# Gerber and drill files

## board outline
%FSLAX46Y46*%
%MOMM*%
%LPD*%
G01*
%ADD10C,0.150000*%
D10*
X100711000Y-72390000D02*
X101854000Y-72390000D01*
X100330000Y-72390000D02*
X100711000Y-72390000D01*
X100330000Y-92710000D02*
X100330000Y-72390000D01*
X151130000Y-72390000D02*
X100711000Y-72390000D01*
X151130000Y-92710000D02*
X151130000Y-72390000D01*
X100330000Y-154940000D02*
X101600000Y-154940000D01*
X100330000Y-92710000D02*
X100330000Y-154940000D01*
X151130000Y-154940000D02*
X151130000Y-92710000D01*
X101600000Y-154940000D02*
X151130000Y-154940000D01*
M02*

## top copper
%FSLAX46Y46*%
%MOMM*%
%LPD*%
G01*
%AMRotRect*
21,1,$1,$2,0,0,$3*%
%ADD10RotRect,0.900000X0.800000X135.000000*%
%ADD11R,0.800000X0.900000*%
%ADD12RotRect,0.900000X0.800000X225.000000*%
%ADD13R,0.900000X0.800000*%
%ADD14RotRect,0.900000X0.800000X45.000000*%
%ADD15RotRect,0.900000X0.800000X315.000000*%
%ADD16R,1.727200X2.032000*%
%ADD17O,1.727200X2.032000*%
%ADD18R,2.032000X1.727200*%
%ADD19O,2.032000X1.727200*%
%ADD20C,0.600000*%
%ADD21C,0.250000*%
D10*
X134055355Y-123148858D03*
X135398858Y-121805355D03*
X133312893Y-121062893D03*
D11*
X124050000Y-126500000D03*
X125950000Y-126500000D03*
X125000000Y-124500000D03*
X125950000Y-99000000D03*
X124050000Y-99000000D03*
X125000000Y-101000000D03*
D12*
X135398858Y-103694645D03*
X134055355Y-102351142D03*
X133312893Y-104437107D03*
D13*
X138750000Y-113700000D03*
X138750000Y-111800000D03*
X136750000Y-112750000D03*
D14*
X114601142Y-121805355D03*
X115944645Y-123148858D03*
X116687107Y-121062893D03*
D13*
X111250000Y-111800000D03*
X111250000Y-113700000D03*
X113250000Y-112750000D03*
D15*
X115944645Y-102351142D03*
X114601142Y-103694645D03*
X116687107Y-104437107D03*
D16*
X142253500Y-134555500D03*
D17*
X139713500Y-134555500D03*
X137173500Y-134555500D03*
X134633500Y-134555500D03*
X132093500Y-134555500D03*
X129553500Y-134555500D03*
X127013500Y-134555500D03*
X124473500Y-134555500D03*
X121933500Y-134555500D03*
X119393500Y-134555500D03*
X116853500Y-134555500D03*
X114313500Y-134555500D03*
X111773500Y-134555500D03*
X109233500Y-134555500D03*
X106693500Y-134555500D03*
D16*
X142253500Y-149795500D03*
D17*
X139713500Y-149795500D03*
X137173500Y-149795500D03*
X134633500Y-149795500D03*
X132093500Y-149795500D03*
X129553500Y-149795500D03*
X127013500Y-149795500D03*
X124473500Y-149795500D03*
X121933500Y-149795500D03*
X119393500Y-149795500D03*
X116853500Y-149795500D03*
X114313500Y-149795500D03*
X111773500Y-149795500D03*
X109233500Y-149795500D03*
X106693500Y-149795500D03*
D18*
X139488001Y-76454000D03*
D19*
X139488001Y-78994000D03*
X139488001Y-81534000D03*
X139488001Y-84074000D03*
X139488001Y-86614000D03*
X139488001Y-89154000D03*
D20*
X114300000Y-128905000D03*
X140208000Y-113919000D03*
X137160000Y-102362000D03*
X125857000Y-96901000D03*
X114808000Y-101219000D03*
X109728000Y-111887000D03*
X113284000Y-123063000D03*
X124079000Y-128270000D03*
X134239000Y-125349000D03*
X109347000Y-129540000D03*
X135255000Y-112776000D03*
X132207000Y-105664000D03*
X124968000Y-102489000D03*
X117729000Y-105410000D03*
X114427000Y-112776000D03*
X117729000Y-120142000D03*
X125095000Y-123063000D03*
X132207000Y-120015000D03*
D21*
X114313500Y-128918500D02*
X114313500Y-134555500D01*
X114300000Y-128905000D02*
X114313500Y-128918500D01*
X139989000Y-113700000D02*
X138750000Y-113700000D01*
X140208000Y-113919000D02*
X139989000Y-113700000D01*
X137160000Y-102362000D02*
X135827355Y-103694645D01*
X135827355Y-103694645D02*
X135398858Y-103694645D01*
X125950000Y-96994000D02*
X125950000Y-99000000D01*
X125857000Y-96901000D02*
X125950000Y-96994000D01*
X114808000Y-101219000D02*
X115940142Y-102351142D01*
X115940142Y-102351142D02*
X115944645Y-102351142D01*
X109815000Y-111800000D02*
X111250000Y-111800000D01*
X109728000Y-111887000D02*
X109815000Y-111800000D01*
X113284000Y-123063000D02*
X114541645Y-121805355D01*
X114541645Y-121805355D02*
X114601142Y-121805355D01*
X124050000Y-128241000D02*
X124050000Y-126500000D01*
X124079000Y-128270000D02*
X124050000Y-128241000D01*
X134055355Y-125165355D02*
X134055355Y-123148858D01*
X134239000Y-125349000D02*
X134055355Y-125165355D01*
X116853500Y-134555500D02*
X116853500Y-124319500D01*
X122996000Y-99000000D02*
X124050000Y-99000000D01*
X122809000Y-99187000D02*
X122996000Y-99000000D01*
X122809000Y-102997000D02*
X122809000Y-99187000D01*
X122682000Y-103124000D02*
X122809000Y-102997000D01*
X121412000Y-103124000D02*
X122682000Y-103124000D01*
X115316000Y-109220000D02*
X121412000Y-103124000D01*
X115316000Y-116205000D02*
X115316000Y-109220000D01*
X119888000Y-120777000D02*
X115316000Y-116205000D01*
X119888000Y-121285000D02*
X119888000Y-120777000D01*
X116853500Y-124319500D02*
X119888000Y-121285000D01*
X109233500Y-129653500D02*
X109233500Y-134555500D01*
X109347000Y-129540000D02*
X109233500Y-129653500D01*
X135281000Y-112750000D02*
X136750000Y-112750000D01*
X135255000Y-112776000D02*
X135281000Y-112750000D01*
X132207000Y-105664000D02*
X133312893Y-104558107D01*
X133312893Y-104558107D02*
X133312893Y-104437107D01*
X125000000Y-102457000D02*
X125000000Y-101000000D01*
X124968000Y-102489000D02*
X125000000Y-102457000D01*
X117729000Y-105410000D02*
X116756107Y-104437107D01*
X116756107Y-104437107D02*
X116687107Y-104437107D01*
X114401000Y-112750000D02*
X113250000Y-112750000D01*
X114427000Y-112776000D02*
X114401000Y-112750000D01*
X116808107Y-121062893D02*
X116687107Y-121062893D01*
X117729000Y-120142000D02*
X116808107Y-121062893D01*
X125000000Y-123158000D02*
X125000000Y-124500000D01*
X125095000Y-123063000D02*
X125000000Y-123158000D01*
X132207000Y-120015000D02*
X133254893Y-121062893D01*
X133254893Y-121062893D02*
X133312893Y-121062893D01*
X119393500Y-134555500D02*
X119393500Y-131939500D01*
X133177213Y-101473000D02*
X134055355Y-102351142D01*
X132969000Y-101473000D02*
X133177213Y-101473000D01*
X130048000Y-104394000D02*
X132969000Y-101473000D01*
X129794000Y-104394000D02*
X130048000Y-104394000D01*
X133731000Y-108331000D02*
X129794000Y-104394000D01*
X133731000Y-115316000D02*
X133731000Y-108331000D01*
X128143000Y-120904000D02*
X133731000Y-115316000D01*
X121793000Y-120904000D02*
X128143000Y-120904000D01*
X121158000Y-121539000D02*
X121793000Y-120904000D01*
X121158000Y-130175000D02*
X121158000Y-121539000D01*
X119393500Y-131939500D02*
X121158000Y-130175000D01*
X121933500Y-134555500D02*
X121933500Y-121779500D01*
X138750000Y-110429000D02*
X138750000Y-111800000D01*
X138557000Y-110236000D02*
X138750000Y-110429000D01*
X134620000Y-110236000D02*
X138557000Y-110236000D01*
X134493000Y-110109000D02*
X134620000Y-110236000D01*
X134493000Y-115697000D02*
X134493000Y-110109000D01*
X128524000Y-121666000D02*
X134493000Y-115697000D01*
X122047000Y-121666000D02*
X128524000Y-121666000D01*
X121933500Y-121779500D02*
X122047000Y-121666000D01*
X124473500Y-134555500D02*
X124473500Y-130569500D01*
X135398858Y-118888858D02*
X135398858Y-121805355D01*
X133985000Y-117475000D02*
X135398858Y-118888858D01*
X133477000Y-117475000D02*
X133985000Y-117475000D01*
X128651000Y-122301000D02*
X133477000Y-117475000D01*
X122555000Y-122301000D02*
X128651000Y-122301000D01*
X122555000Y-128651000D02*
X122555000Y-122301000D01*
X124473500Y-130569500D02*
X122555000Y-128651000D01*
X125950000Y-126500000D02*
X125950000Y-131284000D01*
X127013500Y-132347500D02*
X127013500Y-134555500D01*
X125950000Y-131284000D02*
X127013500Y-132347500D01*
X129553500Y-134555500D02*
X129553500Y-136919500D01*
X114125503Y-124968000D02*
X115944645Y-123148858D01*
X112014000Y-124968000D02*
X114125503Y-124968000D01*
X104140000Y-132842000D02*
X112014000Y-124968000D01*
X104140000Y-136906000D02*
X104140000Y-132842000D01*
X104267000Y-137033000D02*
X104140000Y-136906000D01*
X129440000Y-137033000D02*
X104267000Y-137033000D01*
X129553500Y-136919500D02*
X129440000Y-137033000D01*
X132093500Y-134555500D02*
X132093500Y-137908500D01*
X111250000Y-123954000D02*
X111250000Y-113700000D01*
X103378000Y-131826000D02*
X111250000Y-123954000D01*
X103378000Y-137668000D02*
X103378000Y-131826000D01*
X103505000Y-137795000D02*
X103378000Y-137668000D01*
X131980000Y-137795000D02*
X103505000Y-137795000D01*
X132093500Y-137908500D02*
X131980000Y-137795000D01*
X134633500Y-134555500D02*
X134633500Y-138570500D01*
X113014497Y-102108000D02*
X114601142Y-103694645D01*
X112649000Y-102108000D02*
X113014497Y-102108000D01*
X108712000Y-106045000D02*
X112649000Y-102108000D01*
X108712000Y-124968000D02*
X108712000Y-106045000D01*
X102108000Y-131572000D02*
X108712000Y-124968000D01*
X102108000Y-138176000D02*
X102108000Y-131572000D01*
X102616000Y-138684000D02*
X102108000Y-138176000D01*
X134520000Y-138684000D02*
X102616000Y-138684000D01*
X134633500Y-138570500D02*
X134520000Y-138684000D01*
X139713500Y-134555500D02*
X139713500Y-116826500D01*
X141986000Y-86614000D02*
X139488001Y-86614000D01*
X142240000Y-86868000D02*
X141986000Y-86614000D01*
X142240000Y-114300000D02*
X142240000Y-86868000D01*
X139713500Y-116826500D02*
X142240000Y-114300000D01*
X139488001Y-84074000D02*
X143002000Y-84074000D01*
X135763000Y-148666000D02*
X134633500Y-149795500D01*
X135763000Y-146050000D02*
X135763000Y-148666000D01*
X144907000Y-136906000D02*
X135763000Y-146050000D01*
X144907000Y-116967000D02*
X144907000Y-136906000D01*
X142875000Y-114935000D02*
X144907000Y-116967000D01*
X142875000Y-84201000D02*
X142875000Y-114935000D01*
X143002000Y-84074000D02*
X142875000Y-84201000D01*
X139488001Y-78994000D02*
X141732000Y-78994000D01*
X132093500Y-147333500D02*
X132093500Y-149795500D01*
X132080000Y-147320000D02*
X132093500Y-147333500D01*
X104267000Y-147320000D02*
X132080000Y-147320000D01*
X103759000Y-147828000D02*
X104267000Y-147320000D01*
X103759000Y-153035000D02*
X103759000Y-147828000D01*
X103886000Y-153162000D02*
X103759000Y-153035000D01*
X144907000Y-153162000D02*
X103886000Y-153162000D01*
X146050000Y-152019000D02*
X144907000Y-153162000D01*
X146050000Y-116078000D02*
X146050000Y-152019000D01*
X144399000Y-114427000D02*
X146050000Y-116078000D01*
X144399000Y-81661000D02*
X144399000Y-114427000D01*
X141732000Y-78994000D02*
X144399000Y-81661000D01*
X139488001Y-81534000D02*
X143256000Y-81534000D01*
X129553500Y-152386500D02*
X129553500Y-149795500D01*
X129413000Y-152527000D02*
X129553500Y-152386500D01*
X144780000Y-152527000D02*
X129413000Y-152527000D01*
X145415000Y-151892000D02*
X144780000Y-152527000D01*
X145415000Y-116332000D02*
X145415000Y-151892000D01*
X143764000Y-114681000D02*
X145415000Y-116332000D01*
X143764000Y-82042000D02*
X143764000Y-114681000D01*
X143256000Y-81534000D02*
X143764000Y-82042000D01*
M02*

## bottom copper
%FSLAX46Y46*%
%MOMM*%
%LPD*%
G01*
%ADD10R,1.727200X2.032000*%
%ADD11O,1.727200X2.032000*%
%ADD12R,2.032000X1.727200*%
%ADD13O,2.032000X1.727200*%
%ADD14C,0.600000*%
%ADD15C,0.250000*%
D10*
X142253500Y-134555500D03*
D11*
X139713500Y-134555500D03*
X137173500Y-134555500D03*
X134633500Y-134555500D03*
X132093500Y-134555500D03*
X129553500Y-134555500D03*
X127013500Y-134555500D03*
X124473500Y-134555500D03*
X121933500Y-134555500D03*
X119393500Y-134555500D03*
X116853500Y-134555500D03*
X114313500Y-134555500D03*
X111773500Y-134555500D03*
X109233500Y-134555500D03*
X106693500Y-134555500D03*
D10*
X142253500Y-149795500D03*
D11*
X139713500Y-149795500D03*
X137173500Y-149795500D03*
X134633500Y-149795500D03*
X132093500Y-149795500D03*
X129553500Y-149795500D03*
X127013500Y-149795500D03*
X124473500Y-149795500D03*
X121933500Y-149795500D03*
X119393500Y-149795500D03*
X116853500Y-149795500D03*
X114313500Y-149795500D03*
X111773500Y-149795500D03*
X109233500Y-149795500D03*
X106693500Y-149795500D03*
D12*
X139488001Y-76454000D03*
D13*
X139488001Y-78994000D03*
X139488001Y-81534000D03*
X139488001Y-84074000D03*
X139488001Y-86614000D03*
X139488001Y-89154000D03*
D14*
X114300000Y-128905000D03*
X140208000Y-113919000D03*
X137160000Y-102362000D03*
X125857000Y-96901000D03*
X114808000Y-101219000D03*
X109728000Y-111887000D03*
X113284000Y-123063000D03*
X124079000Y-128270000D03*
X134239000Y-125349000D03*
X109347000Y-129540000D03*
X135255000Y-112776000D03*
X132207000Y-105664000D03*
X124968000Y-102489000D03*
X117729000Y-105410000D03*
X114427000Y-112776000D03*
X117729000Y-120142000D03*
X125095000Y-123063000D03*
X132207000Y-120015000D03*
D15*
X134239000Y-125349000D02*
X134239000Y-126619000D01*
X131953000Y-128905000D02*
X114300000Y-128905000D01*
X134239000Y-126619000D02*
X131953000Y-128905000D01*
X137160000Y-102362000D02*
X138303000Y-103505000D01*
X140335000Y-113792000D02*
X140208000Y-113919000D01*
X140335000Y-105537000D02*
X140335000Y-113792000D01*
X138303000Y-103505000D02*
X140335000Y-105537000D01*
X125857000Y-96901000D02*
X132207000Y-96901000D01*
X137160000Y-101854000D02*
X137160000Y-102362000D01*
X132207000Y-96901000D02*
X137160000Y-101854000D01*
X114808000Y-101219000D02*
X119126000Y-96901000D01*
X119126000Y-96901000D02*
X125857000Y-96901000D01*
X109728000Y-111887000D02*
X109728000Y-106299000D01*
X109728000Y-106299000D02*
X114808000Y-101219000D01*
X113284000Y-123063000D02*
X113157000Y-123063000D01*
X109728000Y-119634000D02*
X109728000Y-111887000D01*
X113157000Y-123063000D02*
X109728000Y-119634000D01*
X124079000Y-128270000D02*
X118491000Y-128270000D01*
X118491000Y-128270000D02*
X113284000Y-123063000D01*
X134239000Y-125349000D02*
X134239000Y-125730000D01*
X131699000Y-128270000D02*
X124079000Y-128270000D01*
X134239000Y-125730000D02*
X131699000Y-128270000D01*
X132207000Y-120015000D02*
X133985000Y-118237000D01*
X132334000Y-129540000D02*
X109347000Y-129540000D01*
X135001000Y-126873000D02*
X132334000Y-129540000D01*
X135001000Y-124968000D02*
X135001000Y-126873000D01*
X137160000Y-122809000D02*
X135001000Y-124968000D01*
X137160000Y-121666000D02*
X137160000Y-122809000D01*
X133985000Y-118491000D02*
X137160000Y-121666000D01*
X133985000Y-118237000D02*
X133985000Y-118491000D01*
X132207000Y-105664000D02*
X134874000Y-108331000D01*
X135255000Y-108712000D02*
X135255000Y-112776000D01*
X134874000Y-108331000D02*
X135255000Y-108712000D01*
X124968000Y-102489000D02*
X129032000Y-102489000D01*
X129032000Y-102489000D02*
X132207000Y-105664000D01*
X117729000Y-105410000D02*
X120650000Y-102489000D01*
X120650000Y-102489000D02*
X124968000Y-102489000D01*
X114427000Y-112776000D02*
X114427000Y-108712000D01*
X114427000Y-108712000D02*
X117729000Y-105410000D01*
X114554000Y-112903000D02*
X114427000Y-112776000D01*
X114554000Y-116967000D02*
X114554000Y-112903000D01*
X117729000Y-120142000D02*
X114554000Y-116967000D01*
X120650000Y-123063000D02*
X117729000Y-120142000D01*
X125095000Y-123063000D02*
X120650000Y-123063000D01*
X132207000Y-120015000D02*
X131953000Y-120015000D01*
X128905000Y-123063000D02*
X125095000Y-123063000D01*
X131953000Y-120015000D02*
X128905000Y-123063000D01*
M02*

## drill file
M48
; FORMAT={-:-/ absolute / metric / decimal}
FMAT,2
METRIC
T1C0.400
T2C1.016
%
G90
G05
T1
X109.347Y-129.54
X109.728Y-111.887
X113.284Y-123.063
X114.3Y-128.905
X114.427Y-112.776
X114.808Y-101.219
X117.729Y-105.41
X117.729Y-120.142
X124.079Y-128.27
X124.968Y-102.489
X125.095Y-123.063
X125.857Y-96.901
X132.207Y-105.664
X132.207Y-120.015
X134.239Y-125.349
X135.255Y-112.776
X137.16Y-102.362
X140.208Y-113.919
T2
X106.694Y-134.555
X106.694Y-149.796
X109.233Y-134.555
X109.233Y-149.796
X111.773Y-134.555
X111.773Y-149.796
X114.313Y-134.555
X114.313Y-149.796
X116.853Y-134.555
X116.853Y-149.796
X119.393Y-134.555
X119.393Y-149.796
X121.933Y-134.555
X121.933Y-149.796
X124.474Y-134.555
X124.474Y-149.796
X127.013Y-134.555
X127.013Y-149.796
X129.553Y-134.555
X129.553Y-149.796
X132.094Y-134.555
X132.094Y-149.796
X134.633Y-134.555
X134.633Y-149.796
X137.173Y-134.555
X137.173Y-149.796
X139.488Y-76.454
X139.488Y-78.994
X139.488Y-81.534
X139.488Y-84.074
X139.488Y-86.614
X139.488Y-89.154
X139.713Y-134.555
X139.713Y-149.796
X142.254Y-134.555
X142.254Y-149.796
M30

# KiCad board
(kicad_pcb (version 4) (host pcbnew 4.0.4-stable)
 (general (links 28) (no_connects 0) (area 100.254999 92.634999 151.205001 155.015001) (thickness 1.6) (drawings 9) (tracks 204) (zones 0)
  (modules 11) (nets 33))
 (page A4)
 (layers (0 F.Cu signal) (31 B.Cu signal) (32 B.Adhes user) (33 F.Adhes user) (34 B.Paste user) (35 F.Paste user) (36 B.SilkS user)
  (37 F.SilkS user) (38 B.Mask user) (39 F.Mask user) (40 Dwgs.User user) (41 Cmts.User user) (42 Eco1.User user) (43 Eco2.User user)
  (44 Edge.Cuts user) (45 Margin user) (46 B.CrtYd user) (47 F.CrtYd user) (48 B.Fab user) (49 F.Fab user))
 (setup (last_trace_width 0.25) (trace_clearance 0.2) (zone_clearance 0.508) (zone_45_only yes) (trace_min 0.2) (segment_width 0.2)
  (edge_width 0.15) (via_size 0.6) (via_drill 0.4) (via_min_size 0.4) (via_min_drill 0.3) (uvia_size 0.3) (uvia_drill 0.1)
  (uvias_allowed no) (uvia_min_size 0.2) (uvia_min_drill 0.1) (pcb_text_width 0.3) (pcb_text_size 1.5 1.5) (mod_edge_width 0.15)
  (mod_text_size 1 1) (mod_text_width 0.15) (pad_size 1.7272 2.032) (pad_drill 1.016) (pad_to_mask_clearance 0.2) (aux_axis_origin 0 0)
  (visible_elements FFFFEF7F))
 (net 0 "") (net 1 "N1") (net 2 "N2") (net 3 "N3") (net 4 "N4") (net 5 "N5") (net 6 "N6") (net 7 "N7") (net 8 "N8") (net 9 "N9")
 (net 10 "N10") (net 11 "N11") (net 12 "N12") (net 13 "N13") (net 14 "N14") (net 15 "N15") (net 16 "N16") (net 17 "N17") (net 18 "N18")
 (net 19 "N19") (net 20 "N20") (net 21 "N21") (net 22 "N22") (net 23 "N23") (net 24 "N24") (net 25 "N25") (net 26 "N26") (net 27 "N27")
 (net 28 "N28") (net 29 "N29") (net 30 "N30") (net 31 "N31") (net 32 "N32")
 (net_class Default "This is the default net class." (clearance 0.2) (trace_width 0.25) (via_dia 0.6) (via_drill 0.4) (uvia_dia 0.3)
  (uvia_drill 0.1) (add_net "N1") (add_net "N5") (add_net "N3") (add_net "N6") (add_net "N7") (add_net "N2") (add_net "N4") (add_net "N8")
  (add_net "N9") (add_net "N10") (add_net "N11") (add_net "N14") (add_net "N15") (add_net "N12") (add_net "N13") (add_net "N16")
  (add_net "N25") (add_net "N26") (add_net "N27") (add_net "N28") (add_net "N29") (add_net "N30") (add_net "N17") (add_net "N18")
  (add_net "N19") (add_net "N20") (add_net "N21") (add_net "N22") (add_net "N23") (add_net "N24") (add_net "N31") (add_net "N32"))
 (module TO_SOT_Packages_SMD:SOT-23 (layer F.Cu) (at 134.02 121.77 135)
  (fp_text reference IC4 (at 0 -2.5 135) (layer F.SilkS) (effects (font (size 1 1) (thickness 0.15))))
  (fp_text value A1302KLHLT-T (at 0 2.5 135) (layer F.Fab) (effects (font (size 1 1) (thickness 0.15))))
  (pad 1 smd rect (at -1 -0.95 135) (size 0.9 0.8) (layers F.Cu F.Paste F.Mask) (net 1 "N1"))
  (pad 2 smd rect (at -1 0.95 135) (size 0.9 0.8) (layers F.Cu F.Paste F.Mask) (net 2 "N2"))
  (pad 3 smd rect (at 1 0 135) (size 0.9 0.8) (layers F.Cu F.Paste F.Mask) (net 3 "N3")))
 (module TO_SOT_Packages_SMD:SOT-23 (layer F.Cu) (at 125 125.5 90)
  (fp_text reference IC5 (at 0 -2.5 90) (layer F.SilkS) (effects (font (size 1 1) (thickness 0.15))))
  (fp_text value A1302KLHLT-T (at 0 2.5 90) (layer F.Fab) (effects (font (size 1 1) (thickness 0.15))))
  (pad 1 smd rect (at -1 -0.95 90) (size 0.9 0.8) (layers F.Cu F.Paste F.Mask) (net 1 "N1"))
  (pad 2 smd rect (at -1 0.95 90) (size 0.9 0.8) (layers F.Cu F.Paste F.Mask) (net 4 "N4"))
  (pad 3 smd rect (at 1 0 90) (size 0.9 0.8) (layers F.Cu F.Paste F.Mask) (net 3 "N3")))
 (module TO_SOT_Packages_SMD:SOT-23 (layer F.Cu) (at 125 100 270)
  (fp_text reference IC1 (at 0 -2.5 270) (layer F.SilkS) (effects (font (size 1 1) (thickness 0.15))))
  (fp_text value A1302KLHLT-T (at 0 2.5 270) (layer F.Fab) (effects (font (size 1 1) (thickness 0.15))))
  (pad 1 smd rect (at -1 -0.95 270) (size 0.9 0.8) (layers F.Cu F.Paste F.Mask) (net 1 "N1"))
  (pad 2 smd rect (at -1 0.95 270) (size 0.9 0.8) (layers F.Cu F.Paste F.Mask) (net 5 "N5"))
  (pad 3 smd rect (at 1 0 270) (size 0.9 0.8) (layers F.Cu F.Paste F.Mask) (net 3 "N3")))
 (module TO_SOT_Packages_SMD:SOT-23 (layer F.Cu) (at 134.02 103.73 225)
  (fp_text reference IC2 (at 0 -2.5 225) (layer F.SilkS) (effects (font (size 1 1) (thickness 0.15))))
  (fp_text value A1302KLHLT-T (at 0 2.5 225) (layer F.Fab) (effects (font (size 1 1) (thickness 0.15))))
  (pad 1 smd rect (at -1 -0.95 225) (size 0.9 0.8) (layers F.Cu F.Paste F.Mask) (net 1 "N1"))
  (pad 2 smd rect (at -1 0.95 225) (size 0.9 0.8) (layers F.Cu F.Paste F.Mask) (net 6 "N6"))
  (pad 3 smd rect (at 1 0 225) (size 0.9 0.8) (layers F.Cu F.Paste F.Mask) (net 3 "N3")))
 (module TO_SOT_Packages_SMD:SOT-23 (layer F.Cu) (at 137.75 112.75 180)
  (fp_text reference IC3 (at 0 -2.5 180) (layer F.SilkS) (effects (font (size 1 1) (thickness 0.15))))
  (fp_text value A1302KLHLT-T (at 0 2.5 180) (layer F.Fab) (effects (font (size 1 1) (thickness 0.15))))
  (pad 1 smd rect (at -1 -0.95 180) (size 0.9 0.8) (layers F.Cu F.Paste F.Mask) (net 1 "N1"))
  (pad 2 smd rect (at -1 0.95 180) (size 0.9 0.8) (layers F.Cu F.Paste F.Mask) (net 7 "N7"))
  (pad 3 smd rect (at 1 0 180) (size 0.9 0.8) (layers F.Cu F.Paste F.Mask) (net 3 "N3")))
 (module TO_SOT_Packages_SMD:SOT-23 (layer F.Cu) (at 115.98 121.77 45)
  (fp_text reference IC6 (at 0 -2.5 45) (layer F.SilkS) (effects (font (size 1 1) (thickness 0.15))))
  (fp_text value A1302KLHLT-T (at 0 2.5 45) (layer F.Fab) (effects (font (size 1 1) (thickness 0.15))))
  (pad 1 smd rect (at -1 -0.95 45) (size 0.9 0.8) (layers F.Cu F.Paste F.Mask) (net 1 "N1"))
  (pad 2 smd rect (at -1 0.95 45) (size 0.9 0.8) (layers F.Cu F.Paste F.Mask) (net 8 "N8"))
  (pad 3 smd rect (at 1 0 45) (size 0.9 0.8) (layers F.Cu F.Paste F.Mask) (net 3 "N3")))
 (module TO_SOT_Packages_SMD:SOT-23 (layer F.Cu) (at 112.25 112.75)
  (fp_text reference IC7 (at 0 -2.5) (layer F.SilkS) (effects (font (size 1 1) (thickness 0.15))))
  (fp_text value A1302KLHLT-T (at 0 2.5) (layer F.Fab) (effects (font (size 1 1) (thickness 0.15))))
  (pad 1 smd rect (at -1 -0.95) (size 0.9 0.8) (layers F.Cu F.Paste F.Mask) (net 1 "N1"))
  (pad 2 smd rect (at -1 0.95) (size 0.9 0.8) (layers F.Cu F.Paste F.Mask) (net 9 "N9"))
  (pad 3 smd rect (at 1 0) (size 0.9 0.8) (layers F.Cu F.Paste F.Mask) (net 3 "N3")))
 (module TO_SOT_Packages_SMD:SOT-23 (layer F.Cu) (at 115.98 103.73 315)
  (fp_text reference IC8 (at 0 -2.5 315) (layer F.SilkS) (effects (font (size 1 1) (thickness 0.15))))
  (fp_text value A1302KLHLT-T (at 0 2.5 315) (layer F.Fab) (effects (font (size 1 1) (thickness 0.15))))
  (pad 1 smd rect (at -1 -0.95 315) (size 0.9 0.8) (layers F.Cu F.Paste F.Mask) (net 1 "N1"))
  (pad 2 smd rect (at -1 0.95 315) (size 0.9 0.8) (layers F.Cu F.Paste F.Mask) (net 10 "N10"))
  (pad 3 smd rect (at 1 0 315) (size 0.9 0.8) (layers F.Cu F.Paste F.Mask) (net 3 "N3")))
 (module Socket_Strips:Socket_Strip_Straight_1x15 (layer B.Cu) (at 142.2535 134.5555 180)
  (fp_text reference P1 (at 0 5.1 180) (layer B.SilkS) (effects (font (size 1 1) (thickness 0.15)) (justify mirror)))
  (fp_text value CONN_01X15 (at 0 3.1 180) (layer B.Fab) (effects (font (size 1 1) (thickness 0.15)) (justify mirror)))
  (pad 1 thru_hole rect (at 0 0 180) (size 1.7272 2.032) (drill 1.016) (layers *.Cu *.Mask) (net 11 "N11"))
  (pad 2 thru_hole oval (at 2.54 0 180) (size 1.7272 2.032) (drill 1.016) (layers *.Cu *.Mask) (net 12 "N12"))
  (pad 3 thru_hole oval (at 5.08 0 180) (size 1.7272 2.032) (drill 1.016) (layers *.Cu *.Mask) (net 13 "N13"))
  (pad 4 thru_hole oval (at 7.62 0 180) (size 1.7272 2.032) (drill 1.016) (layers *.Cu *.Mask) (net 10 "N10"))
  (pad 5 thru_hole oval (at 10.16 0 180) (size 1.7272 2.032) (drill 1.016) (layers *.Cu *.Mask) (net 9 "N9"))
  (pad 6 thru_hole oval (at 12.7 0 180) (size 1.7272 2.032) (drill 1.016) (layers *.Cu *.Mask) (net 8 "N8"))
  (pad 7 thru_hole oval (at 15.24 0 180) (size 1.7272 2.032) (drill 1.016) (layers *.Cu *.Mask) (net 4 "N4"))
  (pad 8 thru_hole oval (at 17.78 0 180) (size 1.7272 2.032) (drill 1.016) (layers *.Cu *.Mask) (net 2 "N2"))
  (pad 9 thru_hole oval (at 20.32 0 180) (size 1.7272 2.032) (drill 1.016) (layers *.Cu *.Mask) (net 7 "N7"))
  (pad 10 thru_hole oval (at 22.86 0 180) (size 1.7272 2.032) (drill 1.016) (layers *.Cu *.Mask) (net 6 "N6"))
  (pad 11 thru_hole oval (at 25.4 0 180) (size 1.7272 2.032) (drill 1.016) (layers *.Cu *.Mask) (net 5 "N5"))
  (pad 12 thru_hole oval (at 27.94 0 180) (size 1.7272 2.032) (drill 1.016) (layers *.Cu *.Mask) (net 1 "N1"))
  (pad 13 thru_hole oval (at 30.48 0 180) (size 1.7272 2.032) (drill 1.016) (layers *.Cu *.Mask) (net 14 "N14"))
  (pad 14 thru_hole oval (at 33.02 0 180) (size 1.7272 2.032) (drill 1.016) (layers *.Cu *.Mask) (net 3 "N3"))
  (pad 15 thru_hole oval (at 35.56 0 180) (size 1.7272 2.032) (drill 1.016) (layers *.Cu *.Mask) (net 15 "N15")))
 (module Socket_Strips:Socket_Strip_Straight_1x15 (layer B.Cu) (at 142.2535 149.7955 180)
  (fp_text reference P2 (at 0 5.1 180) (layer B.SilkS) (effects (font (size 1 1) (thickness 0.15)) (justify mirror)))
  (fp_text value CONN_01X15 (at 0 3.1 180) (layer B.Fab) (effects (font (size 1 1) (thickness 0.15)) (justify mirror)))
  (pad 1 thru_hole rect (at 0 0 180) (size 1.7272 2.032) (drill 1.016) (layers *.Cu *.Mask) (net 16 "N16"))
  (pad 2 thru_hole oval (at 2.54 0 180) (size 1.7272 2.032) (drill 1.016) (layers *.Cu *.Mask) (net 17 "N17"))
  (pad 3 thru_hole oval (at 5.08 0 180) (size 1.7272 2.032) (drill 1.016) (layers *.Cu *.Mask) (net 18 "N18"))
  (pad 4 thru_hole oval (at 7.62 0 180) (size 1.7272 2.032) (drill 1.016) (layers *.Cu *.Mask) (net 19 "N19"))
  (pad 5 thru_hole oval (at 10.16 0 180) (size 1.7272 2.032) (drill 1.016) (layers *.Cu *.Mask) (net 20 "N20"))
  (pad 6 thru_hole oval (at 12.7 0 180) (size 1.7272 2.032) (drill 1.016) (layers *.Cu *.Mask) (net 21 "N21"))
  (pad 7 thru_hole oval (at 15.24 0 180) (size 1.7272 2.032) (drill 1.016) (layers *.Cu *.Mask) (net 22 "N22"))
  (pad 8 thru_hole oval (at 17.78 0 180) (size 1.7272 2.032) (drill 1.016) (layers *.Cu *.Mask) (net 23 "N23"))
  (pad 9 thru_hole oval (at 20.32 0 180) (size 1.7272 2.032) (drill 1.016) (layers *.Cu *.Mask) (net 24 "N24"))
  (pad 10 thru_hole oval (at 22.86 0 180) (size 1.7272 2.032) (drill 1.016) (layers *.Cu *.Mask) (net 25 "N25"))
  (pad 11 thru_hole oval (at 25.4 0 180) (size 1.7272 2.032) (drill 1.016) (layers *.Cu *.Mask) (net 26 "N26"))
  (pad 12 thru_hole oval (at 27.94 0 180) (size 1.7272 2.032) (drill 1.016) (layers *.Cu *.Mask) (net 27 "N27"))
  (pad 13 thru_hole oval (at 30.48 0 180) (size 1.7272 2.032) (drill 1.016) (layers *.Cu *.Mask) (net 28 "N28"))
  (pad 14 thru_hole oval (at 33.02 0 180) (size 1.7272 2.032) (drill 1.016) (layers *.Cu *.Mask) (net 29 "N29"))
  (pad 15 thru_hole oval (at 35.56 0 180) (size 1.7272 2.032) (drill 1.016) (layers *.Cu *.Mask) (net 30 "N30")))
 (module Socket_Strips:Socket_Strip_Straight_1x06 (layer B.Cu) (at 139.488001 76.454 270)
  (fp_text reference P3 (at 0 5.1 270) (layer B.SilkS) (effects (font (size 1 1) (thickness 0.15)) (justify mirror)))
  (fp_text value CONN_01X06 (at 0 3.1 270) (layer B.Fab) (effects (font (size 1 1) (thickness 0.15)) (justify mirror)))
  (pad 1 thru_hole rect (at 0 0 270) (size 1.7272 2.032) (drill 1.016) (layers *.Cu *.Mask) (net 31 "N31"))
  (pad 2 thru_hole oval (at 2.54 0 270) (size 1.7272 2.032) (drill 1.016) (layers *.Cu *.Mask) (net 20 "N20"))
  (pad 3 thru_hole oval (at 5.08 0 270) (size 1.7272 2.032) (drill 1.016) (layers *.Cu *.Mask) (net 21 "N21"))
  (pad 4 thru_hole oval (at 7.62 0 270) (size 1.7272 2.032) (drill 1.016) (layers *.Cu *.Mask) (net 19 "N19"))
  (pad 5 thru_hole oval (at 10.16 0 270) (size 1.7272 2.032) (drill 1.016) (layers *.Cu *.Mask) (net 12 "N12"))
  (pad 6 thru_hole oval (at 12.7 0 270) (size 1.7272 2.032) (drill 1.016) (layers *.Cu *.Mask) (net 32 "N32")))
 (gr_line (start 100.711 72.39) (end 101.854 72.39) (angle 90) (layer Edge.Cuts) (width 0.15))
 (gr_line (start 100.33 72.39) (end 100.711 72.39) (angle 90) (layer Edge.Cuts) (width 0.15))
 (gr_line (start 100.33 92.71) (end 100.33 72.39) (angle 90) (layer Edge.Cuts) (width 0.15))
 (gr_line (start 151.13 72.39) (end 100.711 72.39) (angle 90) (layer Edge.Cuts) (width 0.15))
 (gr_line (start 151.13 92.71) (end 151.13 72.39) (angle 90) (layer Edge.Cuts) (width 0.15))
 (gr_line (start 100.33 154.94) (end 101.6 154.94) (angle 90) (layer Edge.Cuts) (width 0.15))
 (gr_line (start 100.33 92.71) (end 100.33 154.94) (angle 90) (layer Edge.Cuts) (width 0.15))
 (gr_line (start 151.13 154.94) (end 151.13 92.71) (angle 90) (layer Edge.Cuts) (width 0.15))
 (gr_line (start 101.6 154.94) (end 151.13 154.94) (angle 90) (layer Edge.Cuts) (width 0.15))
 (segment (start 134.239 125.349) (end 134.239 126.619) (width 0.25) (layer B.Cu) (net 1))
 (segment (start 114.3135 128.9185) (end 114.3135 134.5555) (width 0.25) (layer F.Cu) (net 1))
 (segment (start 114.3 128.905) (end 114.3135 128.9185) (width 0.25) (layer F.Cu) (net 1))
 (via (at 114.3 128.905) (size 0.6) (drill 0.4) (layers F.Cu B.Cu) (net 1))
 (segment (start 131.953 128.905) (end 114.3 128.905) (width 0.25) (layer B.Cu) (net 1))
 (segment (start 134.239 126.619) (end 131.953 128.905) (width 0.25) (layer B.Cu) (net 1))
 (segment (start 137.16 102.362) (end 138.303 103.505) (width 0.25) (layer B.Cu) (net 1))
 (segment (start 139.989 113.7) (end 138.75 113.7) (width 0.25) (layer F.Cu) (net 1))
 (segment (start 140.208 113.919) (end 139.989 113.7) (width 0.25) (layer F.Cu) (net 1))
 (via (at 140.208 113.919) (size 0.6) (drill 0.4) (layers F.Cu B.Cu) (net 1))
 (segment (start 140.335 113.792) (end 140.208 113.919) (width 0.25) (layer B.Cu) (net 1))
 (segment (start 140.335 105.537) (end 140.335 113.792) (width 0.25) (layer B.Cu) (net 1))
 (segment (start 138.303 103.505) (end 140.335 105.537) (width 0.25) (layer B.Cu) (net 1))
 (segment (start 125.857 96.901) (end 132.207 96.901) (width 0.25) (layer B.Cu) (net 1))
 (segment (start 137.16 102.362) (end 135.827355 103.694645) (width 0.25) (layer F.Cu) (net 1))
 (via (at 137.16 102.362) (size 0.6) (drill 0.4) (layers F.Cu B.Cu) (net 1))
 (segment (start 137.16 101.854) (end 137.16 102.362) (width 0.25) (layer B.Cu) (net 1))
 (segment (start 132.207 96.901) (end 137.16 101.854) (width 0.25) (layer B.Cu) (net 1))
 (segment (start 135.827355 103.694645) (end 135.398858 103.694645) (width 0.25) (layer F.Cu) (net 1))
 (segment (start 114.808 101.219) (end 119.126 96.901) (width 0.25) (layer B.Cu) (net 1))
 (segment (start 125.95 96.994) (end 125.95 99) (width 0.25) (layer F.Cu) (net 1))
 (segment (start 125.857 96.901) (end 125.95 96.994) (width 0.25) (layer F.Cu) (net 1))
 (via (at 125.857 96.901) (size 0.6) (drill 0.4) (layers F.Cu B.Cu) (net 1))
 (segment (start 119.126 96.901) (end 125.857 96.901) (width 0.25) (layer B.Cu) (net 1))
 (segment (start 109.728 111.887) (end 109.728 106.299) (width 0.25) (layer B.Cu) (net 1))
 (segment (start 114.808 101.219) (end 115.940142 102.351142) (width 0.25) (layer F.Cu) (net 1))
 (via (at 114.808 101.219) (size 0.6) (drill 0.4) (layers F.Cu B.Cu) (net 1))
 (segment (start 109.728 106.299) (end 114.808 101.219) (width 0.25) (layer B.Cu) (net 1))
 (segment (start 115.940142 102.351142) (end 115.944645 102.351142) (width 0.25) (layer F.Cu) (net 1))
 (segment (start 113.284 123.063) (end 113.157 123.063) (width 0.25) (layer B.Cu) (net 1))
 (segment (start 109.815 111.8) (end 111.25 111.8) (width 0.25) (layer F.Cu) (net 1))
 (segment (start 109.728 111.887) (end 109.815 111.8) (width 0.25) (layer F.Cu) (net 1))
 (via (at 109.728 111.887) (size 0.6) (drill 0.4) (layers F.Cu B.Cu) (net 1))
 (segment (start 109.728 119.634) (end 109.728 111.887) (width 0.25) (layer B.Cu) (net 1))
 (segment (start 113.157 123.063) (end 109.728 119.634) (width 0.25) (layer B.Cu) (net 1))
 (segment (start 124.079 128.27) (end 118.491 128.27) (width 0.25) (layer B.Cu) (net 1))
 (segment (start 113.284 123.063) (end 114.541645 121.805355) (width 0.25) (layer F.Cu) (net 1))
 (via (at 113.284 123.063) (size 0.6) (drill 0.4) (layers F.Cu B.Cu) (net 1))
 (segment (start 118.491 128.27) (end 113.284 123.063) (width 0.25) (layer B.Cu) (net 1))
 (segment (start 114.541645 121.805355) (end 114.601142 121.805355) (width 0.25) (layer F.Cu) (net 1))
 (segment (start 134.239 125.349) (end 134.239 125.73) (width 0.25) (layer B.Cu) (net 1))
 (segment (start 124.05 128.241) (end 124.05 126.5) (width 0.25) (layer F.Cu) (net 1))
 (segment (start 124.079 128.27) (end 124.05 128.241) (width 0.25) (layer F.Cu) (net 1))
 (via (at 124.079 128.27) (size 0.6) (drill 0.4) (layers F.Cu B.Cu) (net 1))
 (segment (start 131.699 128.27) (end 124.079 128.27) (width 0.25) (layer B.Cu) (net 1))
 (segment (start 134.239 125.73) (end 131.699 128.27) (width 0.25) (layer B.Cu) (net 1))
 (segment (start 134.055355 125.165355) (end 134.055355 123.148858) (width 0.25) (layer F.Cu) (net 1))
 (segment (start 134.239 125.349) (end 134.055355 125.165355) (width 0.25) (layer F.Cu) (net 1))
 (via (at 134.239 125.349) (size 0.6) (drill 0.4) (layers F.Cu B.Cu) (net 1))
 (segment (start 116.8535 134.5555) (end 116.8535 124.3195) (width 0.25) (layer F.Cu) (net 5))
 (segment (start 122.996 99) (end 124.05 99) (width 0.25) (layer F.Cu) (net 5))
 (segment (start 122.809 99.187) (end 122.996 99) (width 0.25) (layer F.Cu) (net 5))
 (segment (start 122.809 102.997) (end 122.809 99.187) (width 0.25) (layer F.Cu) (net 5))
 (segment (start 122.682 103.124) (end 122.809 102.997) (width 0.25) (layer F.Cu) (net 5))
 (segment (start 121.412 103.124) (end 122.682 103.124) (width 0.25) (layer F.Cu) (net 5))
 (segment (start 115.316 109.22) (end 121.412 103.124) (width 0.25) (layer F.Cu) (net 5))
 (segment (start 115.316 116.205) (end 115.316 109.22) (width 0.25) (layer F.Cu) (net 5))
 (segment (start 119.888 120.777) (end 115.316 116.205) (width 0.25) (layer F.Cu) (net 5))
 (segment (start 119.888 121.285) (end 119.888 120.777) (width 0.25) (layer F.Cu) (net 5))
 (segment (start 116.8535 124.3195) (end 119.888 121.285) (width 0.25) (layer F.Cu) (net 5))
 (segment (start 132.207 120.015) (end 133.985 118.237) (width 0.25) (layer B.Cu) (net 3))
 (segment (start 109.2335 129.6535) (end 109.2335 134.5555) (width 0.25) (layer F.Cu) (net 3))
 (segment (start 109.347 129.54) (end 109.2335 129.6535) (width 0.25) (layer F.Cu) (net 3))
 (via (at 109.347 129.54) (size 0.6) (drill 0.4) (layers F.Cu B.Cu) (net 3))
 (segment (start 132.334 129.54) (end 109.347 129.54) (width 0.25) (layer B.Cu) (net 3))
 (segment (start 135.001 126.873) (end 132.334 129.54) (width 0.25) (layer B.Cu) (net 3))
 (segment (start 135.001 124.968) (end 135.001 126.873) (width 0.25) (layer B.Cu) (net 3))
 (segment (start 137.16 122.809) (end 135.001 124.968) (width 0.25) (layer B.Cu) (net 3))
 (segment (start 137.16 121.666) (end 137.16 122.809) (width 0.25) (layer B.Cu) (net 3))
 (segment (start 133.985 118.491) (end 137.16 121.666) (width 0.25) (layer B.Cu) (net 3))
 (segment (start 133.985 118.237) (end 133.985 118.491) (width 0.25) (layer B.Cu) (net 3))
 (segment (start 132.207 105.664) (end 134.874 108.331) (width 0.25) (layer B.Cu) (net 3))
 (segment (start 135.281 112.75) (end 136.75 112.75) (width 0.25) (layer F.Cu) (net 3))
 (segment (start 135.255 112.776) (end 135.281 112.75) (width 0.25) (layer F.Cu) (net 3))
 (via (at 135.255 112.776) (size 0.6) (drill 0.4) (layers F.Cu B.Cu) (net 3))
 (segment (start 135.255 108.712) (end 135.255 112.776) (width 0.25) (layer B.Cu) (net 3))
 (segment (start 134.874 108.331) (end 135.255 108.712) (width 0.25) (layer B.Cu) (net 3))
 (segment (start 124.968 102.489) (end 129.032 102.489) (width 0.25) (layer B.Cu) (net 3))
 (segment (start 132.207 105.664) (end 133.312893 104.558107) (width 0.25) (layer F.Cu) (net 3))
 (via (at 132.207 105.664) (size 0.6) (drill 0.4) (layers F.Cu B.Cu) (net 3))
 (segment (start 129.032 102.489) (end 132.207 105.664) (width 0.25) (layer B.Cu) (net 3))
 (segment (start 133.312893 104.558107) (end 133.312893 104.437107) (width 0.25) (layer F.Cu) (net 3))
 (segment (start 117.729 105.41) (end 120.65 102.489) (width 0.25) (layer B.Cu) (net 3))
 (segment (start 125 102.457) (end 125 101) (width 0.25) (layer F.Cu) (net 3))
 (segment (start 124.968 102.489) (end 125 102.457) (width 0.25) (layer F.Cu) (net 3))
 (via (at 124.968 102.489) (size 0.6) (drill 0.4) (layers F.Cu B.Cu) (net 3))
 (segment (start 120.65 102.489) (end 124.968 102.489) (width 0.25) (layer B.Cu) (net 3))
 (segment (start 114.427 112.776) (end 114.427 108.712) (width 0.25) (layer B.Cu) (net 3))
 (segment (start 117.729 105.41) (end 116.756107 104.437107) (width 0.25) (layer F.Cu) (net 3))
 (via (at 117.729 105.41) (size 0.6) (drill 0.4) (layers F.Cu B.Cu) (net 3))
 (segment (start 114.427 108.712) (end 117.729 105.41) (width 0.25) (layer B.Cu) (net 3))
 (segment (start 116.756107 104.437107) (end 116.687107 104.437107) (width 0.25) (layer F.Cu) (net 3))
 (segment (start 114.401 112.75) (end 113.25 112.75) (width 0.25) (layer F.Cu) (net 3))
 (segment (start 114.427 112.776) (end 114.401 112.75) (width 0.25) (layer F.Cu) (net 3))
 (via (at 114.427 112.776) (size 0.6) (drill 0.4) (layers F.Cu B.Cu) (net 3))
 (segment (start 114.554 112.903) (end 114.427 112.776) (width 0.25) (layer B.Cu) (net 3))
 (segment (start 114.554 116.967) (end 114.554 112.903) (width 0.25) (layer B.Cu) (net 3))
 (segment (start 117.729 120.142) (end 114.554 116.967) (width 0.25) (layer B.Cu) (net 3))
 (segment (start 116.808107 121.062893) (end 116.687107 121.062893) (width 0.25) (layer F.Cu) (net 3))
 (segment (start 117.729 120.142) (end 116.808107 121.062893) (width 0.25) (layer F.Cu) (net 3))
 (via (at 117.729 120.142) (size 0.6) (drill 0.4) (layers F.Cu B.Cu) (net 3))
 (segment (start 120.65 123.063) (end 117.729 120.142) (width 0.25) (layer B.Cu) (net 3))
 (segment (start 125.095 123.063) (end 120.65 123.063) (width 0.25) (layer B.Cu) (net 3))
 (segment (start 132.207 120.015) (end 131.953 120.015) (width 0.25) (layer B.Cu) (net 3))
 (segment (start 125 123.158) (end 125 124.5) (width 0.25) (layer F.Cu) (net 3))
 (segment (start 125.095 123.063) (end 125 123.158) (width 0.25) (layer F.Cu) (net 3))
 (via (at 125.095 123.063) (size 0.6) (drill 0.4) (layers F.Cu B.Cu) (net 3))
 (segment (start 128.905 123.063) (end 125.095 123.063) (width 0.25) (layer B.Cu) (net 3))
 (segment (start 131.953 120.015) (end 128.905 123.063) (width 0.25) (layer B.Cu) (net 3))
 (segment (start 132.207 120.015) (end 133.254893 121.062893) (width 0.25) (layer F.Cu) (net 3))
 (via (at 132.207 120.015) (size 0.6) (drill 0.4) (layers F.Cu B.Cu) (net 3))
 (segment (start 133.254893 121.062893) (end 133.312893 121.062893) (width 0.25) (layer F.Cu) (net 3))
 (segment (start 119.3935 134.5555) (end 119.3935 131.9395) (width 0.25) (layer F.Cu) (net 6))
 (segment (start 133.177213 101.473) (end 134.055355 102.351142) (width 0.25) (layer F.Cu) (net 6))
 (segment (start 132.969 101.473) (end 133.177213 101.473) (width 0.25) (layer F.Cu) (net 6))
 (segment (start 130.048 104.394) (end 132.969 101.473) (width 0.25) (layer F.Cu) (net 6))
 (segment (start 129.794 104.394) (end 130.048 104.394) (width 0.25) (layer F.Cu) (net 6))
 (segment (start 133.731 108.331) (end 129.794 104.394) (width 0.25) (layer F.Cu) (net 6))
 (segment (start 133.731 115.316) (end 133.731 108.331) (width 0.25) (layer F.Cu) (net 6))
 (segment (start 128.143 120.904) (end 133.731 115.316) (width 0.25) (layer F.Cu) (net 6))
 (segment (start 121.793 120.904) (end 128.143 120.904) (width 0.25) (layer F.Cu) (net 6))
 (segment (start 121.158 121.539) (end 121.793 120.904) (width 0.25) (layer F.Cu) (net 6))
 (segment (start 121.158 130.175) (end 121.158 121.539) (width 0.25) (layer F.Cu) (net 6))
 (segment (start 119.3935 131.9395) (end 121.158 130.175) (width 0.25) (layer F.Cu) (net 6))
 (segment (start 121.9335 134.5555) (end 121.9335 121.7795) (width 0.25) (layer F.Cu) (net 7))
 (segment (start 138.75 110.429) (end 138.75 111.8) (width 0.25) (layer F.Cu) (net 7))
 (segment (start 138.557 110.236) (end 138.75 110.429) (width 0.25) (layer F.Cu) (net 7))
 (segment (start 134.62 110.236) (end 138.557 110.236) (width 0.25) (layer F.Cu) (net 7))
 (segment (start 134.493 110.109) (end 134.62 110.236) (width 0.25) (layer F.Cu) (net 7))
 (segment (start 134.493 115.697) (end 134.493 110.109) (width 0.25) (layer F.Cu) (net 7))
 (segment (start 128.524 121.666) (end 134.493 115.697) (width 0.25) (layer F.Cu) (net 7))
 (segment (start 122.047 121.666) (end 128.524 121.666) (width 0.25) (layer F.Cu) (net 7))
 (segment (start 121.9335 121.7795) (end 122.047 121.666) (width 0.25) (layer F.Cu) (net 7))
 (segment (start 124.4735 134.5555) (end 124.4735 130.5695) (width 0.25) (layer F.Cu) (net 2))
 (segment (start 135.398858 118.888858) (end 135.398858 121.805355) (width 0.25) (layer F.Cu) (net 2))
 (segment (start 133.985 117.475) (end 135.398858 118.888858) (width 0.25) (layer F.Cu) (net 2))
 (segment (start 133.477 117.475) (end 133.985 117.475) (width 0.25) (layer F.Cu) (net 2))
 (segment (start 128.651 122.301) (end 133.477 117.475) (width 0.25) (layer F.Cu) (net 2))
 (segment (start 122.555 122.301) (end 128.651 122.301) (width 0.25) (layer F.Cu) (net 2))
 (segment (start 122.555 128.651) (end 122.555 122.301) (width 0.25) (layer F.Cu) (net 2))
 (segment (start 124.4735 130.5695) (end 122.555 128.651) (width 0.25) (layer F.Cu) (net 2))
 (segment (start 125.95 126.5) (end 125.95 131.284) (width 0.25) (layer F.Cu) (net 4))
 (segment (start 127.0135 132.3475) (end 127.0135 134.5555) (width 0.25) (layer F.Cu) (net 4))
 (segment (start 125.95 131.284) (end 127.0135 132.3475) (width 0.25) (layer F.Cu) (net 4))
 (segment (start 129.5535 134.5555) (end 129.5535 136.9195) (width 0.25) (layer F.Cu) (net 8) (status 400000))
 (segment (start 114.125503 124.968) (end 115.944645 123.148858) (width 0.25) (layer F.Cu) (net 8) (status 800000))
 (segment (start 112.014 124.968) (end 114.125503 124.968) (width 0.25) (layer F.Cu) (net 8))
 (segment (start 104.14 132.842) (end 112.014 124.968) (width 0.25) (layer F.Cu) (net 8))
 (segment (start 104.14 136.906) (end 104.14 132.842) (width 0.25) (layer F.Cu) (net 8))
 (segment (start 104.267 137.033) (end 104.14 136.906) (width 0.25) (layer F.Cu) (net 8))
 (segment (start 129.44 137.033) (end 104.267 137.033) (width 0.25) (layer F.Cu) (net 8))
 (segment (start 129.5535 136.9195) (end 129.44 137.033) (width 0.25) (layer F.Cu) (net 8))
 (segment (start 132.0935 134.5555) (end 132.0935 137.9085) (width 0.25) (layer F.Cu) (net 9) (status 400000))
 (segment (start 111.25 123.954) (end 111.25 113.7) (width 0.25) (layer F.Cu) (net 9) (status 800000))
 (segment (start 103.378 131.826) (end 111.25 123.954) (width 0.25) (layer F.Cu) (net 9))
 (segment (start 103.378 137.668) (end 103.378 131.826) (width 0.25) (layer F.Cu) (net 9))
 (segment (start 103.505 137.795) (end 103.378 137.668) (width 0.25) (layer F.Cu) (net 9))
 (segment (start 131.98 137.795) (end 103.505 137.795) (width 0.25) (layer F.Cu) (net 9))
 (segment (start 132.0935 137.9085) (end 131.98 137.795) (width 0.25) (layer F.Cu) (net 9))
 (segment (start 134.6335 134.5555) (end 134.6335 138.5705) (width 0.25) (layer F.Cu) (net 10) (status 400000))
 (segment (start 113.014497 102.108) (end 114.601142 103.694645) (width 0.25) (layer F.Cu) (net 10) (status 800000))
 (segment (start 112.649 102.108) (end 113.014497 102.108) (width 0.25) (layer F.Cu) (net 10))
 (segment (start 108.712 106.045) (end 112.649 102.108) (width 0.25) (layer F.Cu) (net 10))
 (segment (start 108.712 124.968) (end 108.712 106.045) (width 0.25) (layer F.Cu) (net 10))
 (segment (start 102.108 131.572) (end 108.712 124.968) (width 0.25) (layer F.Cu) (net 10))
 (segment (start 102.108 138.176) (end 102.108 131.572) (width 0.25) (layer F.Cu) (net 10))
 (segment (start 102.616 138.684) (end 102.108 138.176) (width 0.25) (layer F.Cu) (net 10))
 (segment (start 134.52 138.684) (end 102.616 138.684) (width 0.25) (layer F.Cu) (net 10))
 (segment (start 134.6335 138.5705) (end 134.52 138.684) (width 0.25) (layer F.Cu) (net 10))
 (segment (start 139.7135 134.5555) (end 139.7135 116.8265) (width 0.25) (layer F.Cu) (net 12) (status 400000))
 (segment (start 141.986 86.614) (end 139.488001 86.614) (width 0.25) (layer F.Cu) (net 12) (status 800000))
 (segment (start 142.24 86.868) (end 141.986 86.614) (width 0.25) (layer F.Cu) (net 12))
 (segment (start 142.24 114.3) (end 142.24 86.868) (width 0.25) (layer F.Cu) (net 12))
 (segment (start 139.7135 116.8265) (end 142.24 114.3) (width 0.25) (layer F.Cu) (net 12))
 (segment (start 139.488001 84.074) (end 143.002 84.074) (width 0.25) (layer F.Cu) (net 19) (status 400000))
 (segment (start 135.763 148.666) (end 134.6335 149.7955) (width 0.25) (layer F.Cu) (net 19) (status 800000))
 (segment (start 135.763 146.05) (end 135.763 148.666) (width 0.25) (layer F.Cu) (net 19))
 (segment (start 144.907 136.906) (end 135.763 146.05) (width 0.25) (layer F.Cu) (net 19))
 (segment (start 144.907 116.967) (end 144.907 136.906) (width 0.25) (layer F.Cu) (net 19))
 (segment (start 142.875 114.935) (end 144.907 116.967) (width 0.25) (layer F.Cu) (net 19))
 (segment (start 142.875 84.201) (end 142.875 114.935) (width 0.25) (layer F.Cu) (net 19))
 (segment (start 143.002 84.074) (end 142.875 84.201) (width 0.25) (layer F.Cu) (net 19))
 (segment (start 139.488001 78.994) (end 141.732 78.994) (width 0.25) (layer F.Cu) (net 20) (status 400000))
 (segment (start 132.0935 147.3335) (end 132.0935 149.7955) (width 0.25) (layer F.Cu) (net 20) (status 800000))
 (segment (start 132.08 147.32) (end 132.0935 147.3335) (width 0.25) (layer F.Cu) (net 20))
 (segment (start 104.267 147.32) (end 132.08 147.32) (width 0.25) (layer F.Cu) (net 20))
 (segment (start 103.759 147.828) (end 104.267 147.32) (width 0.25) (layer F.Cu) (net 20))
 (segment (start 103.759 153.035) (end 103.759 147.828) (width 0.25) (layer F.Cu) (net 20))
 (segment (start 103.886 153.162) (end 103.759 153.035) (width 0.25) (layer F.Cu) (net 20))
 (segment (start 144.907 153.162) (end 103.886 153.162) (width 0.25) (layer F.Cu) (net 20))
 (segment (start 146.05 152.019) (end 144.907 153.162) (width 0.25) (layer F.Cu) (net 20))
 (segment (start 146.05 116.078) (end 146.05 152.019) (width 0.25) (layer F.Cu) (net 20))
 (segment (start 144.399 114.427) (end 146.05 116.078) (width 0.25) (layer F.Cu) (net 20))
 (segment (start 144.399 81.661) (end 144.399 114.427) (width 0.25) (layer F.Cu) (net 20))
 (segment (start 141.732 78.994) (end 144.399 81.661) (width 0.25) (layer F.Cu) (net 20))
 (segment (start 139.488001 81.534) (end 143.256 81.534) (width 0.25) (layer F.Cu) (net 21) (status 400000))
 (segment (start 129.5535 152.3865) (end 129.5535 149.7955) (width 0.25) (layer F.Cu) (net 21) (status 800000))
 (segment (start 129.413 152.527) (end 129.5535 152.3865) (width 0.25) (layer F.Cu) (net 21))
 (segment (start 144.78 152.527) (end 129.413 152.527) (width 0.25) (layer F.Cu) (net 21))
 (segment (start 145.415 151.892) (end 144.78 152.527) (width 0.25) (layer F.Cu) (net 21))
 (segment (start 145.415 116.332) (end 145.415 151.892) (width 0.25) (layer F.Cu) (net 21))
 (segment (start 143.764 114.681) (end 145.415 116.332) (width 0.25) (layer F.Cu) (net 21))
 (segment (start 143.764 82.042) (end 143.764 114.681) (width 0.25) (layer F.Cu) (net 21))
 (segment (start 143.256 81.534) (end 143.764 82.042) (width 0.25) (layer F.Cu) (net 21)))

